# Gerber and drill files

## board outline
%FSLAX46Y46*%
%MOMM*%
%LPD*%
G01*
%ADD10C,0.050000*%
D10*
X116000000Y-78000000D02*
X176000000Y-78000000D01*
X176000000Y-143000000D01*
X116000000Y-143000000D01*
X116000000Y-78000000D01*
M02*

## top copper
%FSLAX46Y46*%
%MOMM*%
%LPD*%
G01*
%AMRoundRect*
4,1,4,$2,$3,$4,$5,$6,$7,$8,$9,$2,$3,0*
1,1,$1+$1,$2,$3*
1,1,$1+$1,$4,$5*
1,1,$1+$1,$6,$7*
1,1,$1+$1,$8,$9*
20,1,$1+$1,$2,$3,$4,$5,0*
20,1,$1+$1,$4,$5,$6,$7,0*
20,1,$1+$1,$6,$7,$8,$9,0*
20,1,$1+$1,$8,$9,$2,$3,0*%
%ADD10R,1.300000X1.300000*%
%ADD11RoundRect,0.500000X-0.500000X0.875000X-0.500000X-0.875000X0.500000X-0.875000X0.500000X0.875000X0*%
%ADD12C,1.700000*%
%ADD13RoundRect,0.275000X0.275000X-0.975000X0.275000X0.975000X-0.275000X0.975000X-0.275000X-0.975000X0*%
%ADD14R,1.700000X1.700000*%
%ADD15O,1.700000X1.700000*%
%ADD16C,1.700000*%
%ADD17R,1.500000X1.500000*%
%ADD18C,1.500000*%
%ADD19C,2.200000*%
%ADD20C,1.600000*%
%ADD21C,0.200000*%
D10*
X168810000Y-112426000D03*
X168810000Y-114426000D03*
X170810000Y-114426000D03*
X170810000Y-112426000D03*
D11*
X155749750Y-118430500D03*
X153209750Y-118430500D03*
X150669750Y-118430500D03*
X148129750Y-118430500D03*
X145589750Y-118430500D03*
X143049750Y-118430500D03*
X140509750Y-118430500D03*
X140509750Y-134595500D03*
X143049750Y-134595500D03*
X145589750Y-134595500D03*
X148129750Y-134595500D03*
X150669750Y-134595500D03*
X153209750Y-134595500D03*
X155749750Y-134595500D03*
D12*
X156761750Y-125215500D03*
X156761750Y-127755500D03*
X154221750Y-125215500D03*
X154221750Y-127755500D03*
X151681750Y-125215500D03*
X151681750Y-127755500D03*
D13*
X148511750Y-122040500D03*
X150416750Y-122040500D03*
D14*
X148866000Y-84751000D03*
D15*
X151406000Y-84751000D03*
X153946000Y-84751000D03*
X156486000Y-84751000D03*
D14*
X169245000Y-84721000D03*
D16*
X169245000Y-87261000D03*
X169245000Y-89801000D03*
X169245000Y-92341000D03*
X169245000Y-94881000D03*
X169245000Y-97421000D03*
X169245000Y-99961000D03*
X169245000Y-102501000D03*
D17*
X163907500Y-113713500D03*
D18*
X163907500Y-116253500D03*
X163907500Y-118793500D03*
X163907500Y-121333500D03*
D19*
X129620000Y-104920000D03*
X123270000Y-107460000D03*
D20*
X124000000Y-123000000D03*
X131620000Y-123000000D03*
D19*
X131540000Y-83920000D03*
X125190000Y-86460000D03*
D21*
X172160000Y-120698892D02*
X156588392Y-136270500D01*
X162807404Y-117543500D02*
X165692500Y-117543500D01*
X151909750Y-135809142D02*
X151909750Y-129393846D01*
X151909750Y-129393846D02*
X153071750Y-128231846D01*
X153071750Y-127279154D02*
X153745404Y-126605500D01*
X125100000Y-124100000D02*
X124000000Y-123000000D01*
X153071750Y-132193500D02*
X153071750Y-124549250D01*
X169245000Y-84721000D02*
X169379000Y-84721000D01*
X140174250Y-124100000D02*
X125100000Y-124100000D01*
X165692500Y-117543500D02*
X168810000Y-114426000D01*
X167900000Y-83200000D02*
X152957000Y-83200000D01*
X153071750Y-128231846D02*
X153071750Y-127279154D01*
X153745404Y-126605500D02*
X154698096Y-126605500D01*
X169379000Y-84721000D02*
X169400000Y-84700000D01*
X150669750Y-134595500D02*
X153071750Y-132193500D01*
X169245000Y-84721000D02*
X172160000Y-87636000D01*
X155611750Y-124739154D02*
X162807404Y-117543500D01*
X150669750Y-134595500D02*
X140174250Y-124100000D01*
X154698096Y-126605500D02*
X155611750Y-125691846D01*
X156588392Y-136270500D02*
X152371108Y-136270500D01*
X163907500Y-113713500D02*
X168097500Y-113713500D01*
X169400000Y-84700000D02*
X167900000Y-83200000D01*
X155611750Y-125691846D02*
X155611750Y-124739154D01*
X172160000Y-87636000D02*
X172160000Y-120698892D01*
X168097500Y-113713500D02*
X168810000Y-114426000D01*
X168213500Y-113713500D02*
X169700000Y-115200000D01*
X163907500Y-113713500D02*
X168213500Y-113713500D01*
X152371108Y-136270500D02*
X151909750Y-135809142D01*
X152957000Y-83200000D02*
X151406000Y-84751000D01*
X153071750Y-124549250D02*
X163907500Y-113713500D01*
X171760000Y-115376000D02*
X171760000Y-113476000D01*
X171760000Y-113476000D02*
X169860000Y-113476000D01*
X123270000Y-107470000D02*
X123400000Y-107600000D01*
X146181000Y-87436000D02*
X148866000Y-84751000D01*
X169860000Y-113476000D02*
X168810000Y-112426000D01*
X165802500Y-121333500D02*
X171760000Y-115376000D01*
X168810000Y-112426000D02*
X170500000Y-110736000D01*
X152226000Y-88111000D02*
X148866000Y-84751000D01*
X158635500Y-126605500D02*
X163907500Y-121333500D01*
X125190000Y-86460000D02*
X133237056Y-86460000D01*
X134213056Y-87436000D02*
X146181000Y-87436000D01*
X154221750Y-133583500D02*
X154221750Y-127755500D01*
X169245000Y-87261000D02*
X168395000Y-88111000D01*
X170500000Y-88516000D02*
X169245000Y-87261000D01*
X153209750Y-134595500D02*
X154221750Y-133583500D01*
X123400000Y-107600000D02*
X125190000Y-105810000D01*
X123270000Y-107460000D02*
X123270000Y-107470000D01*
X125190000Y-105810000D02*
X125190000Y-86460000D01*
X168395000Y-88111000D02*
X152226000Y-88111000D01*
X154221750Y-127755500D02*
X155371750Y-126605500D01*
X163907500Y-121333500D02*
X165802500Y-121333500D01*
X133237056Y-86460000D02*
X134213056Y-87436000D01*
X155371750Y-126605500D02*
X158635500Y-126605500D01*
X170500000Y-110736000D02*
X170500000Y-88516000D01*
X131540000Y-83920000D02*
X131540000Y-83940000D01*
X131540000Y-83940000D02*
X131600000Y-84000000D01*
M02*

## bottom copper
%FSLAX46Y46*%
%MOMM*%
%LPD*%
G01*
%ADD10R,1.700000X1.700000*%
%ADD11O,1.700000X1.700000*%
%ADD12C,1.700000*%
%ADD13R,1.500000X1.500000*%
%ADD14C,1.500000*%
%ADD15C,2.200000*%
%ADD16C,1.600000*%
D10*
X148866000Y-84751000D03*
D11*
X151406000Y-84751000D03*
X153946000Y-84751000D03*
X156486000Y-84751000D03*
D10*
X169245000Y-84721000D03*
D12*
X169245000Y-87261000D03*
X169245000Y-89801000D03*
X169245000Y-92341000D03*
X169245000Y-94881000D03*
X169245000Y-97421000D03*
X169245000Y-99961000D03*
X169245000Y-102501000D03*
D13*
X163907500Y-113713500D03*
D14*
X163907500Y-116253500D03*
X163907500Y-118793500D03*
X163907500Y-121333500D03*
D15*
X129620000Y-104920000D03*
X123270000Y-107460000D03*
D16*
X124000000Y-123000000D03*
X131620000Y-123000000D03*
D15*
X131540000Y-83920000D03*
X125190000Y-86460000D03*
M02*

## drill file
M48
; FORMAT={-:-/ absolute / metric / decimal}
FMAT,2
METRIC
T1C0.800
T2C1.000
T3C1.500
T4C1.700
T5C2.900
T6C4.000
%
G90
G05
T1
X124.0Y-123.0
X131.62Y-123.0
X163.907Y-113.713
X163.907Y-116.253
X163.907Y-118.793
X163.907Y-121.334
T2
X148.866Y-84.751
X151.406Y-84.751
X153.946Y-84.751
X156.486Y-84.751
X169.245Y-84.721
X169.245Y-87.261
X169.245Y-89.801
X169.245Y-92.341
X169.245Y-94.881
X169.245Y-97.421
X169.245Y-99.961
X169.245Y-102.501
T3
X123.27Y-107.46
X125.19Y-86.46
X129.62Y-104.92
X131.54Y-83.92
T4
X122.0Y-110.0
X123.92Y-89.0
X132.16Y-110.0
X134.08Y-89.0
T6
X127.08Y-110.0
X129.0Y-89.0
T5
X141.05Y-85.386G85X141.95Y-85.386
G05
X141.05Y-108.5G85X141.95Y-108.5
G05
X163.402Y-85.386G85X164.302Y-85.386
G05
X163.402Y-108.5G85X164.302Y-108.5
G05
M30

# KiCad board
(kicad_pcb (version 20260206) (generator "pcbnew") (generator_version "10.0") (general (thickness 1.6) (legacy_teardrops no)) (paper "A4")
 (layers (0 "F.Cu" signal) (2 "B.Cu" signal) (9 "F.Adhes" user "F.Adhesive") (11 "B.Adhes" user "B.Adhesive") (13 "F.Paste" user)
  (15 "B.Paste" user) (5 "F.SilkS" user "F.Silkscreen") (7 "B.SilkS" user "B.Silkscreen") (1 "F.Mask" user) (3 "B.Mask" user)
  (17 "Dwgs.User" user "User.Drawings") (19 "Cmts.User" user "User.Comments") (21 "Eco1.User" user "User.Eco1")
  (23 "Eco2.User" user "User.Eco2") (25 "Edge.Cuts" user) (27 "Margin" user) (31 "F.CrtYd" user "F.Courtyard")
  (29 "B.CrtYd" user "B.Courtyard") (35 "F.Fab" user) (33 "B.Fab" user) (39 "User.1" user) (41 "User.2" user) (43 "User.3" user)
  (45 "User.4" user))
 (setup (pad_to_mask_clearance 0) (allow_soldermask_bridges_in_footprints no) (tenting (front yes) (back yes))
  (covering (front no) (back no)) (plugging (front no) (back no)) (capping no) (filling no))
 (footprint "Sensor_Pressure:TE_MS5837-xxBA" (layer "F.Cu") (at 169.81 113.426)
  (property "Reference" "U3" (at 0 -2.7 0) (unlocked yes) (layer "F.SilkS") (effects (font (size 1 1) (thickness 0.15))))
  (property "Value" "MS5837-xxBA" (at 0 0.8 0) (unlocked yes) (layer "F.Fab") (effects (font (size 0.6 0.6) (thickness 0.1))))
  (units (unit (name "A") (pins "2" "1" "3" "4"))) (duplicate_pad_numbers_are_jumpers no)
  (pad "1" smd rect (at -1 -1 180) (size 1.3 1.3) (layers "F.Cu" "F.Mask" "F.Paste") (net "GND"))
  (pad "2" smd rect (at -1 1 180) (size 1.3 1.3) (layers "F.Cu" "F.Mask" "F.Paste") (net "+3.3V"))
  (pad "3" smd rect (at 1 1 180) (size 1.3 1.3) (layers "F.Cu" "F.Mask" "F.Paste") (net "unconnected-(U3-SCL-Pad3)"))
  (pad "4" smd rect (at 1 -1 180) (size 1.3 1.3) (layers "F.Cu" "F.Mask" "F.Paste") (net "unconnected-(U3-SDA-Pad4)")))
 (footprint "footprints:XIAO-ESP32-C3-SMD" (layer "F.Cu") (at 137.62975 117.5955 -90)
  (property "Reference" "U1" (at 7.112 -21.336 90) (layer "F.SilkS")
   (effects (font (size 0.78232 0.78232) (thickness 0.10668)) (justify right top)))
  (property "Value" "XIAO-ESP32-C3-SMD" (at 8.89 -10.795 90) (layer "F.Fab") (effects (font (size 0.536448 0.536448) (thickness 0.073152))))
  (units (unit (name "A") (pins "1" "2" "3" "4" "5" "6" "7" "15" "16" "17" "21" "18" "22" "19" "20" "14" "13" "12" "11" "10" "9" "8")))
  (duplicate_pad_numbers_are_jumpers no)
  (pad "1" smd roundrect (at 0.835 -18.12 270) (size 2.75 2) (layers "F.Cu" "F.Mask" "F.Paste") (roundrect_rratio 0.25)
   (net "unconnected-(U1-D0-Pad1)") (solder_mask_margin 0.0508) (thermal_bridge_angle 45))
  (pad "2" smd roundrect (at 0.835 -15.58 270) (size 2.75 2) (layers "F.Cu" "F.Mask" "F.Paste") (roundrect_rratio 0.25)
   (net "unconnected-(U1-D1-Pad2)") (solder_mask_margin 0.0508) (thermal_bridge_angle 45))
  (pad "3" smd roundrect (at 0.835 -13.04 270) (size 2.75 2) (layers "F.Cu" "F.Mask" "F.Paste") (roundrect_rratio 0.25)
   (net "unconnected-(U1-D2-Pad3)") (solder_mask_margin 0.0508) (thermal_bridge_angle 45))
  (pad "4" smd roundrect (at 0.835 -10.5 270) (size 2.75 2) (layers "F.Cu" "F.Mask" "F.Paste") (roundrect_rratio 0.25)
   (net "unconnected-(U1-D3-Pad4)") (solder_mask_margin 0.0508) (thermal_bridge_angle 45))
  (pad "5" smd roundrect (at 0.835 -7.96 270) (size 2.75 2) (layers "F.Cu" "F.Mask" "F.Paste") (roundrect_rratio 0.25)
   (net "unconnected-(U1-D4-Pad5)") (solder_mask_margin 0.0508) (thermal_bridge_angle 45))
  (pad "6" smd roundrect (at 0.835 -5.42 270) (size 2.75 2) (layers "F.Cu" "F.Mask" "F.Paste") (roundrect_rratio 0.25)
   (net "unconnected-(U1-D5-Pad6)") (solder_mask_margin 0.0508) (thermal_bridge_angle 45))
  (pad "7" smd roundrect (at 0.835 -2.88 270) (size 2.75 2) (layers "F.Cu" "F.Mask" "F.Paste") (roundrect_rratio 0.25)
   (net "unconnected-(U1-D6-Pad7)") (solder_mask_margin 0.0508) (thermal_bridge_angle 45))
  (pad "8" smd roundrect (at 17 -2.88 270) (size 2.75 2) (layers "F.Cu" "F.Mask" "F.Paste") (roundrect_rratio 0.25)
   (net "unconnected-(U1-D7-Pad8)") (solder_mask_margin 0.0508) (thermal_bridge_angle 45))
  (pad "9" smd roundrect (at 17 -5.42 270) (size 2.75 2) (layers "F.Cu" "F.Mask" "F.Paste") (roundrect_rratio 0.25)
   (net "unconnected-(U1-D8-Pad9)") (solder_mask_margin 0.0508) (thermal_bridge_angle 45))
  (pad "10" smd roundrect (at 17 -7.96 270) (size 2.75 2) (layers "F.Cu" "F.Mask" "F.Paste") (roundrect_rratio 0.25)
   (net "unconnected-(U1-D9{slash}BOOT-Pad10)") (solder_mask_margin 0.0508) (thermal_bridge_angle 45))
  (pad "11" smd roundrect (at 17 -10.5 270) (size 2.75 2) (layers "F.Cu" "F.Mask" "F.Paste") (roundrect_rratio 0.25)
   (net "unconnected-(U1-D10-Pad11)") (solder_mask_margin 0.0508) (thermal_bridge_angle 45))
  (pad "12" smd roundrect (at 17 -13.04 270) (size 2.75 2) (layers "F.Cu" "F.Mask" "F.Paste") (roundrect_rratio 0.25) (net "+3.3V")
   (solder_mask_margin 0.0508) (thermal_bridge_angle 45))
  (pad "13" smd roundrect (at 17 -15.58 270) (size 2.75 2) (layers "F.Cu" "F.Mask" "F.Paste") (roundrect_rratio 0.25) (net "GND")
   (solder_mask_margin 0.0508) (thermal_bridge_angle 45))
  (pad "14" smd roundrect (at 17 -18.12 270) (size 2.75 2) (layers "F.Cu" "F.Mask" "F.Paste") (roundrect_rratio 0.25) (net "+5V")
   (solder_mask_margin 0.0508) (thermal_bridge_angle 45))
  (pad "15" smd circle (at 7.62 -19.132 270) (size 1.7 1.7) (layers "F.Cu" "F.Mask" "F.Paste") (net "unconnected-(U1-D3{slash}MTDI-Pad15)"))
  (pad "16" smd circle (at 10.16 -19.132 270) (size 1.7 1.7) (layers "F.Cu" "F.Mask" "F.Paste") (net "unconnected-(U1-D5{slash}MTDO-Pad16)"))
  (pad "17" smd circle (at 7.62 -16.592 270) (size 1.7 1.7) (layers "F.Cu" "F.Mask" "F.Paste") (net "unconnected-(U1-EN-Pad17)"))
  (pad "18" smd circle (at 10.16 -16.592 270) (size 1.7 1.7) (layers "F.Cu" "F.Mask" "F.Paste") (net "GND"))
  (pad "19" smd circle (at 7.62 -14.052 270) (size 1.7 1.7) (layers "F.Cu" "F.Mask" "F.Paste") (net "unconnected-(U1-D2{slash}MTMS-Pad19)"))
  (pad "20" smd circle (at 10.16 -14.052 270) (size 1.7 1.7) (layers "F.Cu" "F.Mask" "F.Paste") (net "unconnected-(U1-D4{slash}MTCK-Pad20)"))
  (pad "21" smd roundrect (at 4.445 -10.882 90) (size 2.5 1.1) (layers "F.Cu" "F.Mask" "F.Paste") (roundrect_rratio 0.25)
   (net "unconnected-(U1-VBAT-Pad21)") (thermal_bridge_angle 45))
  (pad "22" smd roundrect (at 4.445 -12.787 90) (size 2.5 1.1) (layers "F.Cu" "F.Mask" "F.Paste") (roundrect_rratio 0.25)
   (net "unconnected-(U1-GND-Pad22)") (thermal_bridge_angle 45)))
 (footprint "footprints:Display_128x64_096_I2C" (layer "F.Cu") (at 152.676 84.751)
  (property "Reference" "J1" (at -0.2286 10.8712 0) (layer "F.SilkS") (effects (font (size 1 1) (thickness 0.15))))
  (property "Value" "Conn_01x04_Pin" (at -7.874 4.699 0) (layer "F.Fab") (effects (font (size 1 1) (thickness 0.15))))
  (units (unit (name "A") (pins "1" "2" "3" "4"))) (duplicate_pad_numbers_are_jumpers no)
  (pad "" np_thru_hole oval (at -11.176 0.635) (size 3.8 2.9) (drill oval 3.8 2.9) (layers "*.Cu" "*.Mask"))
  (pad "" np_thru_hole oval (at -11.176 23.749) (size 3.8 2.9) (drill oval 3.8 2.9) (layers "*.Cu" "*.Mask"))
  (pad "" np_thru_hole oval (at 11.176 0.635) (size 3.8 2.9) (drill oval 3.8 2.9) (layers "*.Cu" "*.Mask"))
  (pad "" np_thru_hole oval (at 11.176 23.749) (size 3.8 2.9) (drill oval 3.8 2.9) (layers "*.Cu" "*.Mask"))
  (pad "1" thru_hole rect (at -3.81 0 90) (size 1.7 1.7) (drill 1) (layers "*.Cu" "*.Mask") (remove_unused_layers no) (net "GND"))
  (pad "2" thru_hole oval (at -1.27 0 90) (size 1.7 1.7) (drill 1) (layers "*.Cu" "*.Mask") (remove_unused_layers no) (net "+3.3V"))
  (pad "3" thru_hole oval (at 1.27 0 90) (size 1.7 1.7) (drill 1) (layers "*.Cu" "*.Mask") (remove_unused_layers no)
   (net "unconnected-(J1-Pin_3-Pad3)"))
  (pad "4" thru_hole oval (at 3.81 0 90) (size 1.7 1.7) (drill 1) (layers "*.Cu" "*.Mask") (remove_unused_layers no)
   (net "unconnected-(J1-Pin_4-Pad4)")))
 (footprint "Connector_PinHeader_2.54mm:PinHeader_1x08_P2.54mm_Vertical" (layer "F.Cu") (at 169.245 84.721)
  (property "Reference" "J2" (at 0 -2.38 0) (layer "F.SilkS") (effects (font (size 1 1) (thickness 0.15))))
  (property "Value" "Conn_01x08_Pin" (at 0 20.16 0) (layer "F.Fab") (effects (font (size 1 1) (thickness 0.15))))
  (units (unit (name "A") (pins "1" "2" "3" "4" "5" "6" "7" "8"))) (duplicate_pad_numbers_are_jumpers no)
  (pad "1" thru_hole rect (at 0 0) (size 1.7 1.7) (drill 1) (layers "*.Cu" "*.Mask") (remove_unused_layers no) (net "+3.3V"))
  (pad "2" thru_hole circle (at 0 2.54) (size 1.7 1.7) (drill 1) (layers "*.Cu" "*.Mask") (remove_unused_layers no) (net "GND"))
  (pad "3" thru_hole circle (at 0 5.08) (size 1.7 1.7) (drill 1) (layers "*.Cu" "*.Mask") (remove_unused_layers no)
   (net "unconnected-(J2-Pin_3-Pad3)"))
  (pad "4" thru_hole circle (at 0 7.62) (size 1.7 1.7) (drill 1) (layers "*.Cu" "*.Mask") (remove_unused_layers no)
   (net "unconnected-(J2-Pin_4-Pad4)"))
  (pad "5" thru_hole circle (at 0 10.16) (size 1.7 1.7) (drill 1) (layers "*.Cu" "*.Mask") (remove_unused_layers no)
   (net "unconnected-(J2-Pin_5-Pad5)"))
  (pad "6" thru_hole circle (at 0 12.7) (size 1.7 1.7) (drill 1) (layers "*.Cu" "*.Mask") (remove_unused_layers no)
   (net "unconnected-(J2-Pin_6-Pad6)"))
  (pad "7" thru_hole circle (at 0 15.24) (size 1.7 1.7) (drill 1) (layers "*.Cu" "*.Mask") (remove_unused_layers no)
   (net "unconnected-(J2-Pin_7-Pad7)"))
  (pad "8" thru_hole circle (at 0 17.78) (size 1.7 1.7) (drill 1) (layers "*.Cu" "*.Mask") (remove_unused_layers no)
   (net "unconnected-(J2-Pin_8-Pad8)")))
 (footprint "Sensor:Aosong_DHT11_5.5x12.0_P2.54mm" (layer "F.Cu") (at 163.9075 113.7135)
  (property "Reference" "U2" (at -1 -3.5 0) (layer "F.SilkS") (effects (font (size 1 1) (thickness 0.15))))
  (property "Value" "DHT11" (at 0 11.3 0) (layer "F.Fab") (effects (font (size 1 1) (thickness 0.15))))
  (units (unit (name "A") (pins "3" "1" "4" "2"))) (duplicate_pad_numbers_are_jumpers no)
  (pad "1" thru_hole rect (at 0 0) (size 1.5 1.5) (drill 0.8) (layers "*.Cu" "*.Mask") (remove_unused_layers no) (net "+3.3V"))
  (pad "2" thru_hole circle (at 0 2.54) (size 1.5 1.5) (drill 0.8) (layers "*.Cu" "*.Mask") (remove_unused_layers no)
   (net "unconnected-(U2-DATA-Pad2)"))
  (pad "3" thru_hole circle (at 0 5.08) (size 1.5 1.5) (drill 0.8) (layers "*.Cu" "*.Mask") (remove_unused_layers no)
   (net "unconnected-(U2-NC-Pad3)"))
  (pad "4" thru_hole circle (at 0 7.62) (size 1.5 1.5) (drill 0.8) (layers "*.Cu" "*.Mask") (remove_unused_layers no) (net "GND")))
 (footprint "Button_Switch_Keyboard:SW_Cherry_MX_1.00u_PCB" (layer "F.Cu") (at 129.62 104.92)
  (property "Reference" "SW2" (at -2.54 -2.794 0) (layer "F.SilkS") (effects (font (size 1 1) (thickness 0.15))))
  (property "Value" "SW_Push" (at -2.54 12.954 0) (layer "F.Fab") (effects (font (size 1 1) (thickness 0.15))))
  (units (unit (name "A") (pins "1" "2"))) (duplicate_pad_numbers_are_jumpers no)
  (pad "" np_thru_hole circle (at -7.62 5.08) (size 1.7 1.7) (drill 1.7) (layers "*.Cu" "*.Mask"))
  (pad "" np_thru_hole circle (at -2.54 5.08) (size 4 4) (drill 4) (layers "*.Cu" "*.Mask"))
  (pad "" np_thru_hole circle (at 2.54 5.08) (size 1.7 1.7) (drill 1.7) (layers "*.Cu" "*.Mask"))
  (pad "1" thru_hole circle (at 0 0) (size 2.2 2.2) (drill 1.5) (layers "*.Cu" "*.Mask") (remove_unused_layers no)
   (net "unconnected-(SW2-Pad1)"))
  (pad "2" thru_hole circle (at -6.35 2.54) (size 2.2 2.2) (drill 1.5) (layers "*.Cu" "*.Mask") (remove_unused_layers no) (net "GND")))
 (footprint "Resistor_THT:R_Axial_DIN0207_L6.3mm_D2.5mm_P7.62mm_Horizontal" (layer "F.Cu") (at 124 123)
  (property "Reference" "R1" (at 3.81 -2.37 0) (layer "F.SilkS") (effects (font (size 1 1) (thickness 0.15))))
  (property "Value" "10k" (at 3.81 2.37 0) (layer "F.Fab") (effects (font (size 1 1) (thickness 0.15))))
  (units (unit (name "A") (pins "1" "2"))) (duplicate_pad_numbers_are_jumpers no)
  (pad "1" thru_hole circle (at 0 0) (size 1.6 1.6) (drill 0.8) (layers "*.Cu" "*.Mask") (remove_unused_layers no) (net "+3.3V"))
  (pad "2" thru_hole circle (at 7.62 0) (size 1.6 1.6) (drill 0.8) (layers "*.Cu" "*.Mask") (remove_unused_layers no)
   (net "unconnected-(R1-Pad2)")))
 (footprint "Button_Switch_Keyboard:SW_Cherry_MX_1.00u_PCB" (layer "F.Cu") (at 131.54 83.92)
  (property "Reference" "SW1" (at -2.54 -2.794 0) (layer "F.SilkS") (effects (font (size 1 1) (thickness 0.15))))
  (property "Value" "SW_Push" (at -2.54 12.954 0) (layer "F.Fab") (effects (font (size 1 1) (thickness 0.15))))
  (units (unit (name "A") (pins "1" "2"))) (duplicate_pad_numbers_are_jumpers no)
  (pad "" np_thru_hole circle (at -7.62 5.08) (size 1.7 1.7) (drill 1.7) (layers "*.Cu" "*.Mask"))
  (pad "" np_thru_hole circle (at -2.54 5.08) (size 4 4) (drill 4) (layers "*.Cu" "*.Mask"))
  (pad "" np_thru_hole circle (at 2.54 5.08) (size 1.7 1.7) (drill 1.7) (layers "*.Cu" "*.Mask"))
  (pad "1" thru_hole circle (at 0 0) (size 2.2 2.2) (drill 1.5) (layers "*.Cu" "*.Mask") (remove_unused_layers no)
   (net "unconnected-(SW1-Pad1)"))
  (pad "2" thru_hole circle (at -6.35 2.54) (size 2.2 2.2) (drill 1.5) (layers "*.Cu" "*.Mask") (remove_unused_layers no) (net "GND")))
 (gr_rect (start 116 78) (end 176 143) (stroke (width 0.05) (type default)) (fill no) (layer "Edge.Cuts"))
 (segment (start 172.16 120.698892) (end 156.588392 136.2705) (width 0.2) (layer "F.Cu") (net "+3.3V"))
 (segment (start 162.807404 117.5435) (end 165.6925 117.5435) (width 0.2) (layer "F.Cu") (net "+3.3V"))
 (segment (start 151.90975 135.809142) (end 151.90975 129.393846) (width 0.2) (layer "F.Cu") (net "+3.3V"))
 (segment (start 151.90975 129.393846) (end 153.07175 128.231846) (width 0.2) (layer "F.Cu") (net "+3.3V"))
 (segment (start 153.07175 127.279154) (end 153.745404 126.6055) (width 0.2) (layer "F.Cu") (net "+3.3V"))
 (segment (start 125.1 124.1) (end 124 123) (width 0.2) (layer "F.Cu") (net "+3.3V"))
 (segment (start 153.07175 132.1935) (end 153.07175 124.54925) (width 0.2) (layer "F.Cu") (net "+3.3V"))
 (segment (start 169.245 84.721) (end 169.379 84.721) (width 0.2) (layer "F.Cu") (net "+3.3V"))
 (segment (start 140.17425 124.1) (end 125.1 124.1) (width 0.2) (layer "F.Cu") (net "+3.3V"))
 (segment (start 165.6925 117.5435) (end 168.81 114.426) (width 0.2) (layer "F.Cu") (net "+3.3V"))
 (segment (start 167.9 83.2) (end 152.957 83.2) (width 0.2) (layer "F.Cu") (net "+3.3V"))
 (segment (start 153.07175 128.231846) (end 153.07175 127.279154) (width 0.2) (layer "F.Cu") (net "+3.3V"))
 (segment (start 153.745404 126.6055) (end 154.698096 126.6055) (width 0.2) (layer "F.Cu") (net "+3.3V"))
 (segment (start 169.379 84.721) (end 169.4 84.7) (width 0.2) (layer "F.Cu") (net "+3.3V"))
 (segment (start 150.66975 134.5955) (end 153.07175 132.1935) (width 0.2) (layer "F.Cu") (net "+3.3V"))
 (segment (start 169.245 84.721) (end 172.16 87.636) (width 0.2) (layer "F.Cu") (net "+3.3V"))
 (segment (start 155.61175 124.739154) (end 162.807404 117.5435) (width 0.2) (layer "F.Cu") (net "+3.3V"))
 (segment (start 150.66975 134.5955) (end 140.17425 124.1) (width 0.2) (layer "F.Cu") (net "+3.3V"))
 (segment (start 154.698096 126.6055) (end 155.61175 125.691846) (width 0.2) (layer "F.Cu") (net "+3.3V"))
 (segment (start 156.588392 136.2705) (end 152.371108 136.2705) (width 0.2) (layer "F.Cu") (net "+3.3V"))
 (segment (start 163.9075 113.7135) (end 168.0975 113.7135) (width 0.2) (layer "F.Cu") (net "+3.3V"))
 (segment (start 169.4 84.7) (end 167.9 83.2) (width 0.2) (layer "F.Cu") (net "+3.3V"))
 (segment (start 155.61175 125.691846) (end 155.61175 124.739154) (width 0.2) (layer "F.Cu") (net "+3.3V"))
 (segment (start 172.16 87.636) (end 172.16 120.698892) (width 0.2) (layer "F.Cu") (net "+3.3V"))
 (segment (start 168.0975 113.7135) (end 168.81 114.426) (width 0.2) (layer "F.Cu") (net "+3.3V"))
 (segment (start 168.2135 113.7135) (end 169.7 115.2) (width 0.2) (layer "F.Cu") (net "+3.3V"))
 (segment (start 163.9075 113.7135) (end 168.2135 113.7135) (width 0.2) (layer "F.Cu") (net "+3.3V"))
 (segment (start 152.371108 136.2705) (end 151.90975 135.809142) (width 0.2) (layer "F.Cu") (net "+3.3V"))
 (segment (start 152.957 83.2) (end 151.406 84.751) (width 0.2) (layer "F.Cu") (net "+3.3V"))
 (segment (start 153.07175 124.54925) (end 163.9075 113.7135) (width 0.2) (layer "F.Cu") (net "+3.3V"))
 (segment (start 171.76 115.376) (end 171.76 113.476) (width 0.2) (layer "F.Cu") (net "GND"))
 (segment (start 171.76 113.476) (end 169.86 113.476) (width 0.2) (layer "F.Cu") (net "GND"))
 (segment (start 123.27 107.47) (end 123.4 107.6) (width 0.2) (layer "F.Cu") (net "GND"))
 (segment (start 146.181 87.436) (end 148.866 84.751) (width 0.2) (layer "F.Cu") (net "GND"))
 (segment (start 169.86 113.476) (end 168.81 112.426) (width 0.2) (layer "F.Cu") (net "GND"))
 (segment (start 165.8025 121.3335) (end 171.76 115.376) (width 0.2) (layer "F.Cu") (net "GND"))
 (segment (start 168.81 112.426) (end 170.5 110.736) (width 0.2) (layer "F.Cu") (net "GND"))
 (segment (start 152.226 88.111) (end 148.866 84.751) (width 0.2) (layer "F.Cu") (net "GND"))
 (segment (start 158.6355 126.6055) (end 163.9075 121.3335) (width 0.2) (layer "F.Cu") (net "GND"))
 (segment (start 125.19 86.46) (end 133.237056 86.46) (width 0.2) (layer "F.Cu") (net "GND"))
 (segment (start 134.213056 87.436) (end 146.181 87.436) (width 0.2) (layer "F.Cu") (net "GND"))
 (segment (start 154.22175 133.5835) (end 154.22175 127.7555) (width 0.2) (layer "F.Cu") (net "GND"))
 (segment (start 169.245 87.261) (end 168.395 88.111) (width 0.2) (layer "F.Cu") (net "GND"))
 (segment (start 170.5 88.516) (end 169.245 87.261) (width 0.2) (layer "F.Cu") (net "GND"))
 (segment (start 153.20975 134.5955) (end 154.22175 133.5835) (width 0.2) (layer "F.Cu") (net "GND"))
 (segment (start 123.4 107.6) (end 125.19 105.81) (width 0.2) (layer "F.Cu") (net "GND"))
 (segment (start 123.27 107.46) (end 123.27 107.47) (width 0.2) (layer "F.Cu") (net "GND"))
 (segment (start 125.19 105.81) (end 125.19 86.46) (width 0.2) (layer "F.Cu") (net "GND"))
 (segment (start 168.395 88.111) (end 152.226 88.111) (width 0.2) (layer "F.Cu") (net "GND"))
 (segment (start 154.22175 127.7555) (end 155.37175 126.6055) (width 0.2) (layer "F.Cu") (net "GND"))
 (segment (start 163.9075 121.3335) (end 165.8025 121.3335) (width 0.2) (layer "F.Cu") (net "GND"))
 (segment (start 133.237056 86.46) (end 134.213056 87.436) (width 0.2) (layer "F.Cu") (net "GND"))
 (segment (start 155.37175 126.6055) (end 158.6355 126.6055) (width 0.2) (layer "F.Cu") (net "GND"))
 (segment (start 170.5 110.736) (end 170.5 88.516) (width 0.2) (layer "F.Cu") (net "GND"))
 (segment (start 131.54 83.92) (end 131.54 83.94) (width 0.2) (layer "F.Cu") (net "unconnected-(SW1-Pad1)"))
 (segment (start 131.54 83.94) (end 131.6 84) (width 0.2) (layer "F.Cu") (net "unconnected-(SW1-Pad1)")))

